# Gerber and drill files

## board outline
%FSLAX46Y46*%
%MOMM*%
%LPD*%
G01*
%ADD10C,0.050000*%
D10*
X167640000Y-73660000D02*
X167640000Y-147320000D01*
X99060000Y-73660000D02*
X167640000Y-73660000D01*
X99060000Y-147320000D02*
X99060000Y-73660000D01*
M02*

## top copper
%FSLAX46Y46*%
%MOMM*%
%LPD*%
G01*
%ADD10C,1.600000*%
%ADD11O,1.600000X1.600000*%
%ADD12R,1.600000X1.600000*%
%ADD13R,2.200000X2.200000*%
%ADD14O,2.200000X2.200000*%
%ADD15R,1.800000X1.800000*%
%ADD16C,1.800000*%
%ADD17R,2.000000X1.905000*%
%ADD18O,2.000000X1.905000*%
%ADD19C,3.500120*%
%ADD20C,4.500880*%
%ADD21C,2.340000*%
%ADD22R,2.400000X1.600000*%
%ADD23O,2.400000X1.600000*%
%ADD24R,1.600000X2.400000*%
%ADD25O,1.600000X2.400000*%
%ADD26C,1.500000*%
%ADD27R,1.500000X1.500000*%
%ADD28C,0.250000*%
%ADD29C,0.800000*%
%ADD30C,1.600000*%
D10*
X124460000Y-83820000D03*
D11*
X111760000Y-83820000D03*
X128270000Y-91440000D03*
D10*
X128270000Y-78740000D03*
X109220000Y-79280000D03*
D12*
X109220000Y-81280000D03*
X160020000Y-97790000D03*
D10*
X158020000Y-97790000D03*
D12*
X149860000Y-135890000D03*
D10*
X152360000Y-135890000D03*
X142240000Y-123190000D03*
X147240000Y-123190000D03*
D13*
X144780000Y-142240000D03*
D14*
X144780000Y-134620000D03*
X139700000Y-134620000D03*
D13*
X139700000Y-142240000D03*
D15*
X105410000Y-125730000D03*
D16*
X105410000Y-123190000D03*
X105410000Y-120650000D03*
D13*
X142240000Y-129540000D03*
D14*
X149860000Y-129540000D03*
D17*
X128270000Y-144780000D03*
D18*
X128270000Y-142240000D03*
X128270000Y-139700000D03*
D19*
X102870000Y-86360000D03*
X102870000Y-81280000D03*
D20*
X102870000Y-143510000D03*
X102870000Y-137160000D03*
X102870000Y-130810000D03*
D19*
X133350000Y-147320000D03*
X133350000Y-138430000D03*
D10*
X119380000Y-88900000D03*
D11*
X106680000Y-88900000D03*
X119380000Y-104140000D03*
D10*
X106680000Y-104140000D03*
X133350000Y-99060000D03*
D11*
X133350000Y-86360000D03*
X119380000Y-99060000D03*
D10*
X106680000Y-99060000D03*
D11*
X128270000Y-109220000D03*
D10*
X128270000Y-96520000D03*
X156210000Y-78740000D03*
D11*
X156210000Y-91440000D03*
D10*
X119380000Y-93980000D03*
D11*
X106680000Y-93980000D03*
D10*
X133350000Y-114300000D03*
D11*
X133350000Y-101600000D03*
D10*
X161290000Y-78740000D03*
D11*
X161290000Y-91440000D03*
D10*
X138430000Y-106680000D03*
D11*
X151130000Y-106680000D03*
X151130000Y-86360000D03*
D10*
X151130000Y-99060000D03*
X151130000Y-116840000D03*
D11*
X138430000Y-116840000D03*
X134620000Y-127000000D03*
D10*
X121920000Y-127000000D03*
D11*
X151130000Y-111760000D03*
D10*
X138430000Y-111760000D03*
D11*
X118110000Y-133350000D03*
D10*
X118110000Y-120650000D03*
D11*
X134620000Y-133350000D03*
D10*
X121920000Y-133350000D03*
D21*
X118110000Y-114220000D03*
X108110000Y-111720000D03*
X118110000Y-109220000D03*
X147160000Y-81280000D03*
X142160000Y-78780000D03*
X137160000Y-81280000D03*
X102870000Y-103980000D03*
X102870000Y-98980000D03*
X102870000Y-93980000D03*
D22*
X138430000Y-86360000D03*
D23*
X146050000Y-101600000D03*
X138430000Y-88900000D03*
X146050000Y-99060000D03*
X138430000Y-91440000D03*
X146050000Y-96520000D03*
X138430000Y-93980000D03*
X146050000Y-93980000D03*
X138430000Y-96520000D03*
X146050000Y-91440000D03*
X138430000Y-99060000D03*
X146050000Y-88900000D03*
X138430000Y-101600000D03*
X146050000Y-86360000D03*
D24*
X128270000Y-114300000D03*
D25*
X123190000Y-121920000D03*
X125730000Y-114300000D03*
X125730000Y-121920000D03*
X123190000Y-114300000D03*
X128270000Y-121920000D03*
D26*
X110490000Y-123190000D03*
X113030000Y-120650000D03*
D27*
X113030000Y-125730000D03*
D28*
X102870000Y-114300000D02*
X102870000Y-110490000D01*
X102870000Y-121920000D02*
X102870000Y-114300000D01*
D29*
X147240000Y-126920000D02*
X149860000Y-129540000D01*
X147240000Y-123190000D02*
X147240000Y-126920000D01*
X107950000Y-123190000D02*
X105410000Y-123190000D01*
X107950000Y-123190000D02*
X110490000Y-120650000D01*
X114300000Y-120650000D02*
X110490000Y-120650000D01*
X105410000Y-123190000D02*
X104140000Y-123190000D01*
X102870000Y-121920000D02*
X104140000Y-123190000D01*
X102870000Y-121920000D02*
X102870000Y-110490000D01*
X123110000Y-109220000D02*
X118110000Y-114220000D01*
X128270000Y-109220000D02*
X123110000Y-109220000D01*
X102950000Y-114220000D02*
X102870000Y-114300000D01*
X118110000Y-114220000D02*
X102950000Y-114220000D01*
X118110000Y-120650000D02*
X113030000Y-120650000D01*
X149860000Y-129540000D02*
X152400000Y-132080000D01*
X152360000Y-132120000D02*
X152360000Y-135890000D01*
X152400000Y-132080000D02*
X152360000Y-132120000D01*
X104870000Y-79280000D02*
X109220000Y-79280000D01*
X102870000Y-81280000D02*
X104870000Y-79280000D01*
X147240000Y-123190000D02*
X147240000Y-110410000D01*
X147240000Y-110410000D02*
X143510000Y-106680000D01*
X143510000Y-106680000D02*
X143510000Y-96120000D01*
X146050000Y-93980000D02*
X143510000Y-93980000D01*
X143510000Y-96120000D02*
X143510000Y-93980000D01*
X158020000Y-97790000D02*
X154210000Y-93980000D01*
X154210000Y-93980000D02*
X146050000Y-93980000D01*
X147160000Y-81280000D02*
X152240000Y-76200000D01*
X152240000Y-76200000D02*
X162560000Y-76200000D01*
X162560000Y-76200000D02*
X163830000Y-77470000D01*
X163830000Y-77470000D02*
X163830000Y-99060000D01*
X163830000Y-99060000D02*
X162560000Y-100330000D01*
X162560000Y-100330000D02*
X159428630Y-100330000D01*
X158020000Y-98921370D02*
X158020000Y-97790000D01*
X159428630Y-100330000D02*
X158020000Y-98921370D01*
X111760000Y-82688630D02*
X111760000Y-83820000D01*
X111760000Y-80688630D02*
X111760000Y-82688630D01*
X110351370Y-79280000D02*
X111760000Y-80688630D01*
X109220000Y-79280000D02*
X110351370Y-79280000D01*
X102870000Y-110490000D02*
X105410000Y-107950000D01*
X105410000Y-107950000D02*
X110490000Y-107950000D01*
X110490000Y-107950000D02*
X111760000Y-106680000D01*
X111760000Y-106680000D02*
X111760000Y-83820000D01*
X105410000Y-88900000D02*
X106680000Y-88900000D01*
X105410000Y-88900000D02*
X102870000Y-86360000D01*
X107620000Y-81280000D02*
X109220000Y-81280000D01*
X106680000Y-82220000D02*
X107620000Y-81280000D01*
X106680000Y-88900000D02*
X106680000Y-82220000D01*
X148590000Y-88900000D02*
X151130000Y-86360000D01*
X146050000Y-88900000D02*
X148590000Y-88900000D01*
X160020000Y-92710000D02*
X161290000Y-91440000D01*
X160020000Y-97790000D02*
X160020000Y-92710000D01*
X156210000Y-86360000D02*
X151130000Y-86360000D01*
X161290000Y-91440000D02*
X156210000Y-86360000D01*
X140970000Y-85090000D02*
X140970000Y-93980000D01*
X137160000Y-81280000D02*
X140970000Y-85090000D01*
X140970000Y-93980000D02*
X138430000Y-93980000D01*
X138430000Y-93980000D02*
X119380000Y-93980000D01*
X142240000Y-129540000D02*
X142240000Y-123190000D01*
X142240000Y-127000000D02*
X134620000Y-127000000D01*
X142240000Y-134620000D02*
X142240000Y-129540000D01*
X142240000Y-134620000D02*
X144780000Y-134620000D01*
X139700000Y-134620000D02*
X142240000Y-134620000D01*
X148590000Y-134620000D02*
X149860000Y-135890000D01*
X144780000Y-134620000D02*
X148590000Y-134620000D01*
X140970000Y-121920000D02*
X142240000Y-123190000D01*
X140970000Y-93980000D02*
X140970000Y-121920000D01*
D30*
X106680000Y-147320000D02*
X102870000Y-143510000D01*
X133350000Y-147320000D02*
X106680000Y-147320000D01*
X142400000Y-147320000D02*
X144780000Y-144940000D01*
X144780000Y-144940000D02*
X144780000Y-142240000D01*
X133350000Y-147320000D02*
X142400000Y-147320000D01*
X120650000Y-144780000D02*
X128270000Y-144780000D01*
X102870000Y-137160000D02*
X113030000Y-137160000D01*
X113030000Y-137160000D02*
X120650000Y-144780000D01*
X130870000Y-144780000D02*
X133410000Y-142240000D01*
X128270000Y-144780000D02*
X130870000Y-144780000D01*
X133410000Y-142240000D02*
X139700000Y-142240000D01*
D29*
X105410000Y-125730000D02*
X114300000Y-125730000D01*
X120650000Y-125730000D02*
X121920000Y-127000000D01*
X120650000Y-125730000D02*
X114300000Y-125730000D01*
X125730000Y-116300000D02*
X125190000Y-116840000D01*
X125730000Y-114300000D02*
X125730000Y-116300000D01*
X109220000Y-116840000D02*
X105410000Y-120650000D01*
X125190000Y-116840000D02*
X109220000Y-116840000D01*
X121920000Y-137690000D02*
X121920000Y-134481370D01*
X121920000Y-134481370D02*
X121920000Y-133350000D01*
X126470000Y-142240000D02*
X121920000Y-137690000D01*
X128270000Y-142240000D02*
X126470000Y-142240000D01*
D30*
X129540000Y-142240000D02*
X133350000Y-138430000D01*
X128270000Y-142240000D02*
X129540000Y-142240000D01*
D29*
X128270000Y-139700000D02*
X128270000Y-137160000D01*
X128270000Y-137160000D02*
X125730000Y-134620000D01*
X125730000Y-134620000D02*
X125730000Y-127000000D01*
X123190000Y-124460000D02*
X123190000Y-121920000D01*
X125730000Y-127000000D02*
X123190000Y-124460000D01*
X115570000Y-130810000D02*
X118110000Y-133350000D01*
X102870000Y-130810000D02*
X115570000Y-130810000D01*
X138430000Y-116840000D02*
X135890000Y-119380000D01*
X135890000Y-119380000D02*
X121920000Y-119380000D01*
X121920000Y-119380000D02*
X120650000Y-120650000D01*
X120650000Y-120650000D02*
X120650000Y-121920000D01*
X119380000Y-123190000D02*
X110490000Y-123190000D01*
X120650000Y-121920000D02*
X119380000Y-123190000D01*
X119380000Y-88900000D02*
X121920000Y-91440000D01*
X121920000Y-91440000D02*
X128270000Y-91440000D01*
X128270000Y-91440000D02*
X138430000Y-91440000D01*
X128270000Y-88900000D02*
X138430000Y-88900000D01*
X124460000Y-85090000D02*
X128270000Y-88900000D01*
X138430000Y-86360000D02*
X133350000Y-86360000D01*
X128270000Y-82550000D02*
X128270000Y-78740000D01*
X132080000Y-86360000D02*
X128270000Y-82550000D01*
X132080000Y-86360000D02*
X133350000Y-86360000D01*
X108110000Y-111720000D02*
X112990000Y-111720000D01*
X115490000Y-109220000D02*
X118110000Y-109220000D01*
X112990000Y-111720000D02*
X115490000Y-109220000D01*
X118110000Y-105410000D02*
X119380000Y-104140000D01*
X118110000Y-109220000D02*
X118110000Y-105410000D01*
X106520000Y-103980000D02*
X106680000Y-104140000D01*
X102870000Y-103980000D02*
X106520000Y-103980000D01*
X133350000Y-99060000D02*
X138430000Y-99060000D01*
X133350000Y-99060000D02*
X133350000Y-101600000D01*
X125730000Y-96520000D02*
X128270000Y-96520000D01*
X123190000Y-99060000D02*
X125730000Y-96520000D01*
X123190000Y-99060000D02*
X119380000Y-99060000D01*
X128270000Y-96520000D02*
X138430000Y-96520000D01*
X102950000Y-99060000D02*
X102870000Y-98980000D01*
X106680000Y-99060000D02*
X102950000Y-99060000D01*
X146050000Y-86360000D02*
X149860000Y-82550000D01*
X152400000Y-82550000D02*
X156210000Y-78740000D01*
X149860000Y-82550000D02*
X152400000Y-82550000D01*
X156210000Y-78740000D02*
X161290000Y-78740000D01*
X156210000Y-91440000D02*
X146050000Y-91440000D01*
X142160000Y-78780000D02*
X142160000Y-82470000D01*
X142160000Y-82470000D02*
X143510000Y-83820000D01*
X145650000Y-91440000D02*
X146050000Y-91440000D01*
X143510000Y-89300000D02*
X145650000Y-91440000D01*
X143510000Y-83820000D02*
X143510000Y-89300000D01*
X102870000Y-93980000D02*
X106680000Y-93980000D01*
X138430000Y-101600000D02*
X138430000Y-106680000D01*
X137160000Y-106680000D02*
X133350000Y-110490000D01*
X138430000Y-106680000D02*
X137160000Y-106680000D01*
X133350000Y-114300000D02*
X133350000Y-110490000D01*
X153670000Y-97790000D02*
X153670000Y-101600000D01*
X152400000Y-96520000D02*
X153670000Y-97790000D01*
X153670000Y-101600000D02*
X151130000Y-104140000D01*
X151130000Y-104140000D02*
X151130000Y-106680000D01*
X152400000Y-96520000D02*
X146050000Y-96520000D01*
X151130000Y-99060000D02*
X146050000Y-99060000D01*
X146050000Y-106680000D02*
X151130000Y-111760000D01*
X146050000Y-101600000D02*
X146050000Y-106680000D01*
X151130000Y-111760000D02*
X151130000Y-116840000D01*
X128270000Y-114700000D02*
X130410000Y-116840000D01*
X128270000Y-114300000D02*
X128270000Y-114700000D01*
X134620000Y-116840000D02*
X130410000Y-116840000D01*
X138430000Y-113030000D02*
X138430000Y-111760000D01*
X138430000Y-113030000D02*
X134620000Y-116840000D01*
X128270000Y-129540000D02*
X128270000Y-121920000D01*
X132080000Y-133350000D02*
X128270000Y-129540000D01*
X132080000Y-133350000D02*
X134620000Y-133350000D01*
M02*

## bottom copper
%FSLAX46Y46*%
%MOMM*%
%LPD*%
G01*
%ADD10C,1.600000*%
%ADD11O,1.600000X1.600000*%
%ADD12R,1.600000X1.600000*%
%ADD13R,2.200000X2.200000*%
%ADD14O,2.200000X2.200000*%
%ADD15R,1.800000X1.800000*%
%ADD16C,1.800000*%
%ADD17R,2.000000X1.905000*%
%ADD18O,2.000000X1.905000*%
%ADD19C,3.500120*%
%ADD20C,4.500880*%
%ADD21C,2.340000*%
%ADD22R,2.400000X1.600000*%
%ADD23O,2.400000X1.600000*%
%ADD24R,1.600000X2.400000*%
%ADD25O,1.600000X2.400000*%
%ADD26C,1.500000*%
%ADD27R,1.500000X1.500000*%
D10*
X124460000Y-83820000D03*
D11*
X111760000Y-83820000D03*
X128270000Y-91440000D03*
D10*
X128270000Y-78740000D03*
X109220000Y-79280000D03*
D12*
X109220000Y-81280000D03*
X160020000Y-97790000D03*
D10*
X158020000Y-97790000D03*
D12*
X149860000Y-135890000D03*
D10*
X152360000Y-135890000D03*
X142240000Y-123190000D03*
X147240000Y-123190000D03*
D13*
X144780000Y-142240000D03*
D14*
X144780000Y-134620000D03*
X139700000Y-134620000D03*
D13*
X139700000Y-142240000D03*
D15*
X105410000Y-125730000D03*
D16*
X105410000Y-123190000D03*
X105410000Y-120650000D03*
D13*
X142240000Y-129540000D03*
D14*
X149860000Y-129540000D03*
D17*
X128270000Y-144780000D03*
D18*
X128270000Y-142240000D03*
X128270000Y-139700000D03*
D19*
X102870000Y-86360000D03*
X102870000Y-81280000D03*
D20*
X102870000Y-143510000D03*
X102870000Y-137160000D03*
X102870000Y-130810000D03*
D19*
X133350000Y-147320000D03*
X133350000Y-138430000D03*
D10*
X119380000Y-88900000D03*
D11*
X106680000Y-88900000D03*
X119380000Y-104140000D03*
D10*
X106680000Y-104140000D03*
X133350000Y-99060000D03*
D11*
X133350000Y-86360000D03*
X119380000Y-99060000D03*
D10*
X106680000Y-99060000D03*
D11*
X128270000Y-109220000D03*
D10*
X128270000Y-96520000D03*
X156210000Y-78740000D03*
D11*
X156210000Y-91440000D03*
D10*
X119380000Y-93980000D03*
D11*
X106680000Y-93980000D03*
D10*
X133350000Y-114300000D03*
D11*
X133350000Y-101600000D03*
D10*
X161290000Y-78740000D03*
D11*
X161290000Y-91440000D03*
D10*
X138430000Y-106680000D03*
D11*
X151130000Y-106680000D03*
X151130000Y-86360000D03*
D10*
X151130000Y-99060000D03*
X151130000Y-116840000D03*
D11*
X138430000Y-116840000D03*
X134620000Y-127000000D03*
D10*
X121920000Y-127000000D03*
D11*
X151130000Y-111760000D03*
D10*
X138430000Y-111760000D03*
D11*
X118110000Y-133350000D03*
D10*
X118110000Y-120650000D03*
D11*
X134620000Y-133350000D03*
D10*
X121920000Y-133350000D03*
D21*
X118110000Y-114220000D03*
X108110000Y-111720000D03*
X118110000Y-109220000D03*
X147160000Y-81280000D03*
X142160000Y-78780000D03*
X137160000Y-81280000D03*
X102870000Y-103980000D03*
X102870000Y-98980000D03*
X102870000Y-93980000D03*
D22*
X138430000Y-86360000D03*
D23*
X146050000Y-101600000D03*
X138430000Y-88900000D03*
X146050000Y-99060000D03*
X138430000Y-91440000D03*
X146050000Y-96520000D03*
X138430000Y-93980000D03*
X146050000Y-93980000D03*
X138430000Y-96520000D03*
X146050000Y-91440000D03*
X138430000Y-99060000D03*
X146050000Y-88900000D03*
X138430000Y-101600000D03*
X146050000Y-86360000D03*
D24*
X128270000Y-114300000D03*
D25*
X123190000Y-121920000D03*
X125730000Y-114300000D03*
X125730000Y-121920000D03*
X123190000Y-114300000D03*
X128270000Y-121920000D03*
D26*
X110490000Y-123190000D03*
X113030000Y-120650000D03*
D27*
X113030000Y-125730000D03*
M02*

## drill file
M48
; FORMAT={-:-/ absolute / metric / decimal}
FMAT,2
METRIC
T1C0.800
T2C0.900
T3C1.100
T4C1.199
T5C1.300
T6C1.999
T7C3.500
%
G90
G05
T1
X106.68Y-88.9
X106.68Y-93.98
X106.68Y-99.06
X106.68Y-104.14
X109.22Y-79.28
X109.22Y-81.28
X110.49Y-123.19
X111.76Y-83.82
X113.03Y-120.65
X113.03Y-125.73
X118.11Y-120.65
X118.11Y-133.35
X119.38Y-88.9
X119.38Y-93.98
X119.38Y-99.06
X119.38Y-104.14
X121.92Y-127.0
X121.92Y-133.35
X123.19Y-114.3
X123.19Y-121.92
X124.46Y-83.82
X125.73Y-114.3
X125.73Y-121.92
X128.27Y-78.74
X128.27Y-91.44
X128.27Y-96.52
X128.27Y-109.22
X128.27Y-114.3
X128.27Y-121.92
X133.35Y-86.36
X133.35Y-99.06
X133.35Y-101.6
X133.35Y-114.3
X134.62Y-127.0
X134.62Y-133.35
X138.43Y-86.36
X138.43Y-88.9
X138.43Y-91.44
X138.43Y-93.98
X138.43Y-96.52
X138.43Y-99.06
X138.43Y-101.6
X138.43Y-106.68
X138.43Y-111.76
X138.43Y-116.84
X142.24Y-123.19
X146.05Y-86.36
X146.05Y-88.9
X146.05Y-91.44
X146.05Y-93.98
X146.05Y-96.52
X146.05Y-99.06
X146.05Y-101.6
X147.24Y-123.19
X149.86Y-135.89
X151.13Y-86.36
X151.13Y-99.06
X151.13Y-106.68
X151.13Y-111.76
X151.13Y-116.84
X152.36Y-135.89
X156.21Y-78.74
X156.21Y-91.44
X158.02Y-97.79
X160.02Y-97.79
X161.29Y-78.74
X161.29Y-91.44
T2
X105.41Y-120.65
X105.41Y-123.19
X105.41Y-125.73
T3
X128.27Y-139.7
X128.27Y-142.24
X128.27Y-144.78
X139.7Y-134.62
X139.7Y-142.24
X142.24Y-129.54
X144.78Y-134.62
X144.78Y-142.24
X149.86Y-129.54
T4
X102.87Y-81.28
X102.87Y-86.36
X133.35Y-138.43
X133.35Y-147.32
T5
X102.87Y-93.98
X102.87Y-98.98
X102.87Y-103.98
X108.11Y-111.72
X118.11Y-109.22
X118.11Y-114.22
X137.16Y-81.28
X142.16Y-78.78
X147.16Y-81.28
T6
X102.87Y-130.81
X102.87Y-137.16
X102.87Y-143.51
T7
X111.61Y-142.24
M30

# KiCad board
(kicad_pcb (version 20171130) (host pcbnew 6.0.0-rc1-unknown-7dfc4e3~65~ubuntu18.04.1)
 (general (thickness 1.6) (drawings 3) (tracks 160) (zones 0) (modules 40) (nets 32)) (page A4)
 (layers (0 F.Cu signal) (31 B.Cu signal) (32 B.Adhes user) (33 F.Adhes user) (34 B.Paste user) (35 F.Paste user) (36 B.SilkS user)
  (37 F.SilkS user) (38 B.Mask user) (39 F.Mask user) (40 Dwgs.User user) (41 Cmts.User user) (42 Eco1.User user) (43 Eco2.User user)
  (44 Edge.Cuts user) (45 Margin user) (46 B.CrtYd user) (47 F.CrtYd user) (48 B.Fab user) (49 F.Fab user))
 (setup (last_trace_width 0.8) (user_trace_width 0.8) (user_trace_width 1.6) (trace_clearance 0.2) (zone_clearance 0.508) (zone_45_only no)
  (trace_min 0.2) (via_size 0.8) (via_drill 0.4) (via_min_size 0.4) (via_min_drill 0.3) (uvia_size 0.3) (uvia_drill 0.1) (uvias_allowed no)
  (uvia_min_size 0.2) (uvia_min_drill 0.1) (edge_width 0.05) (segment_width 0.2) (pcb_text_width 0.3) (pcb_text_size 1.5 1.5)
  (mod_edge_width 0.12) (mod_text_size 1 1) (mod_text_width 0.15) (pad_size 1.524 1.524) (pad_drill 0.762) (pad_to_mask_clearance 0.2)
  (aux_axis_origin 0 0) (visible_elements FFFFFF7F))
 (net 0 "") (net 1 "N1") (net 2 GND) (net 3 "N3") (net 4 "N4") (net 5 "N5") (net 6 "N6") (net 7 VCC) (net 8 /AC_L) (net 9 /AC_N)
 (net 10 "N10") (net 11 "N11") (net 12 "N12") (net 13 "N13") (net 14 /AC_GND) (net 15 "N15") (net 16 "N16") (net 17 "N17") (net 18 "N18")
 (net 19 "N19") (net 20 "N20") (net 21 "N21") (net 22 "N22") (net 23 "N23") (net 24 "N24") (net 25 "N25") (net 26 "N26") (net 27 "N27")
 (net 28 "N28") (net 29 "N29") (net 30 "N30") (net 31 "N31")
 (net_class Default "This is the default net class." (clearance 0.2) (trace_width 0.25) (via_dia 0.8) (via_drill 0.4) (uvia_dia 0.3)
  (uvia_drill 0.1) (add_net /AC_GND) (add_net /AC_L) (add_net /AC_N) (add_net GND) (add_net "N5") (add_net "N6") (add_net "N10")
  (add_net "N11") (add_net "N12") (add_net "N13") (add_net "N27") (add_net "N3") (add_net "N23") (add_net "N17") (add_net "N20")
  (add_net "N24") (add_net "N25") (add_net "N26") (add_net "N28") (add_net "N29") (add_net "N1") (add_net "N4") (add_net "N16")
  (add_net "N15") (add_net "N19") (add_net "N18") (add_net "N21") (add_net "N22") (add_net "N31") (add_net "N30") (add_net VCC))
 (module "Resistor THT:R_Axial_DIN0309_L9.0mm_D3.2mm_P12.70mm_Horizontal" (layer F.Cu) (at 124.46 83.82 180)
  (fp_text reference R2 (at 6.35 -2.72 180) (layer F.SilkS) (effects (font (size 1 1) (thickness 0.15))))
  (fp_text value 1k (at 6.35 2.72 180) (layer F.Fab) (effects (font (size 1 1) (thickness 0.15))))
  (pad 1 thru_hole circle (at 0 0 180) (size 1.6 1.6) (drill 0.8) (layers *.Cu *.Mask) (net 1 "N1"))
  (pad 2 thru_hole oval (at 12.7 0 180) (size 1.6 1.6) (drill 0.8) (layers *.Cu *.Mask) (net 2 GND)))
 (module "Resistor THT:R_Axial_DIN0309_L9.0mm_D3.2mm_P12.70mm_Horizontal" (layer F.Cu) (at 128.27 78.74 270)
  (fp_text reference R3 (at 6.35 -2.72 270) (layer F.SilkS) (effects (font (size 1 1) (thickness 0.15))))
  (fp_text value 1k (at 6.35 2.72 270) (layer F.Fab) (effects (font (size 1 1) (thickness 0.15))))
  (pad 2 thru_hole oval (at 12.7 0 270) (size 1.6 1.6) (drill 0.8) (layers *.Cu *.Mask) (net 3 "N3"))
  (pad 1 thru_hole circle (at 0 0 270) (size 1.6 1.6) (drill 0.8) (layers *.Cu *.Mask) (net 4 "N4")))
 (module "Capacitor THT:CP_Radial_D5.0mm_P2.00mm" (layer F.Cu) (at 109.22 81.28 90)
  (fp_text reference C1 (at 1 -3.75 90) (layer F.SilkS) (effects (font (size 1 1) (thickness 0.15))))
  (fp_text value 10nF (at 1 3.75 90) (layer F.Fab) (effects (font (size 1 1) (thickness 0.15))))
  (pad 2 thru_hole circle (at 2 0 90) (size 1.6 1.6) (drill 0.8) (layers *.Cu *.Mask) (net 2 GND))
  (pad 1 thru_hole rect (at 0 0 90) (size 1.6 1.6) (drill 0.8) (layers *.Cu *.Mask) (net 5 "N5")))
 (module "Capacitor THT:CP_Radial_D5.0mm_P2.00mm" (layer F.Cu) (at 160.02 97.79 180)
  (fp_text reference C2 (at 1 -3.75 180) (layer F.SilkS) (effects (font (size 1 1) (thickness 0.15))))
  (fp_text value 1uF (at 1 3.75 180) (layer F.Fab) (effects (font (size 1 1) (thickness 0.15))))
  (pad 1 thru_hole rect (at 0 0 180) (size 1.6 1.6) (drill 0.8) (layers *.Cu *.Mask) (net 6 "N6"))
  (pad 2 thru_hole circle (at 2 0 180) (size 1.6 1.6) (drill 0.8) (layers *.Cu *.Mask) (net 2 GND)))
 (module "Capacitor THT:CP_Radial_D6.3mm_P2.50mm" (layer F.Cu) (at 149.86 135.89)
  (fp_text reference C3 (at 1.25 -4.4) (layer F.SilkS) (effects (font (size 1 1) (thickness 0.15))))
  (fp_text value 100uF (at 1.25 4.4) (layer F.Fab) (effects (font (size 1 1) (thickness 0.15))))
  (pad 1 thru_hole rect (at 0 0) (size 1.6 1.6) (drill 0.8) (layers *.Cu *.Mask) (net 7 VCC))
  (pad 2 thru_hole circle (at 2.5 0) (size 1.6 1.6) (drill 0.8) (layers *.Cu *.Mask) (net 2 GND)))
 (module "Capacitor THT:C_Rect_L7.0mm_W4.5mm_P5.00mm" (layer F.Cu) (at 142.24 123.19)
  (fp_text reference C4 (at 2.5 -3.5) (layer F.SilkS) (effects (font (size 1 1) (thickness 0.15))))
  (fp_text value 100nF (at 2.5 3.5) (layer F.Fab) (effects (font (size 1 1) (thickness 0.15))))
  (pad 1 thru_hole circle (at 0 0) (size 1.6 1.6) (drill 0.8) (layers *.Cu *.Mask) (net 7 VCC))
  (pad 2 thru_hole circle (at 5 0) (size 1.6 1.6) (drill 0.8) (layers *.Cu *.Mask) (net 2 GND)))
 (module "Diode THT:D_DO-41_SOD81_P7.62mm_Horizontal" (layer F.Cu) (at 144.78 142.24 90)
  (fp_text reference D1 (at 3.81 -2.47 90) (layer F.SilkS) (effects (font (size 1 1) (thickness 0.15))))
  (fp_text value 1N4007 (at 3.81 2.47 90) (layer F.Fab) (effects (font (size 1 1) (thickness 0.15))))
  (pad 1 thru_hole rect (at 0 0 90) (size 2.2 2.2) (drill 1.1) (layers *.Cu *.Mask) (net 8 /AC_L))
  (pad 2 thru_hole oval (at 7.62 0 90) (size 2.2 2.2) (drill 1.1) (layers *.Cu *.Mask) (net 7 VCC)))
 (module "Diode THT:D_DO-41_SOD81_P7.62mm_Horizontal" (layer F.Cu) (at 139.7 142.24 90)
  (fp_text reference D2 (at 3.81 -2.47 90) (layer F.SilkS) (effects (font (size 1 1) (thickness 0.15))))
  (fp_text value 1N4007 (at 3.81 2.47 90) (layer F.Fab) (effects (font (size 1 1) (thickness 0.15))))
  (pad 2 thru_hole oval (at 7.62 0 90) (size 2.2 2.2) (drill 1.1) (layers *.Cu *.Mask) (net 7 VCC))
  (pad 1 thru_hole rect (at 0 0 90) (size 2.2 2.2) (drill 1.1) (layers *.Cu *.Mask) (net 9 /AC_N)))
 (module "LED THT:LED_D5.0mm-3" (layer F.Cu) (at 105.41 125.73 90)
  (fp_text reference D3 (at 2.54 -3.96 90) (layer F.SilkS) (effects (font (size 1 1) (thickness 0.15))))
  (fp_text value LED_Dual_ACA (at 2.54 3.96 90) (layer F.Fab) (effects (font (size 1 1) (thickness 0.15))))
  (pad 1 thru_hole rect (at 0 0 90) (size 1.8 1.8) (drill 0.9) (layers *.Cu *.Mask) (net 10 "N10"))
  (pad 2 thru_hole circle (at 2.54 0 90) (size 1.8 1.8) (drill 0.9) (layers *.Cu *.Mask) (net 2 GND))
  (pad 3 thru_hole circle (at 5.08 0 90) (size 1.8 1.8) (drill 0.9) (layers *.Cu *.Mask) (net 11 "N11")))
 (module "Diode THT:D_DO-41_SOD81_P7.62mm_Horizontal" (layer F.Cu) (at 142.24 129.54)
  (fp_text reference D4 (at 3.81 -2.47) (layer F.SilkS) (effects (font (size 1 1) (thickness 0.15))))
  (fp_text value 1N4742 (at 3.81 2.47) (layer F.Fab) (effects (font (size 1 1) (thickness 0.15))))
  (pad 1 thru_hole rect (at 0 0) (size 2.2 2.2) (drill 1.1) (layers *.Cu *.Mask) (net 7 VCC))
  (pad 2 thru_hole oval (at 7.62 0) (size 2.2 2.2) (drill 1.1) (layers *.Cu *.Mask) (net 2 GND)))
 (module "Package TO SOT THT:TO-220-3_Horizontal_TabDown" (layer F.Cu) (at 128.27 144.78 90)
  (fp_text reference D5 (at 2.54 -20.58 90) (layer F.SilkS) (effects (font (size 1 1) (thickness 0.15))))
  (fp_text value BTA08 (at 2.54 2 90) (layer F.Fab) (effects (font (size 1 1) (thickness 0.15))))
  (pad "" np_thru_hole oval (at 2.54 -16.66 90) (size 3.5 3.5) (drill 3.5) (layers *.Cu *.Mask))
  (pad 1 thru_hole rect (at 0 0 90) (size 1.905 2) (drill 1.1) (layers *.Cu *.Mask) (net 9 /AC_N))
  (pad 2 thru_hole oval (at 2.54 0 90) (size 1.905 2) (drill 1.1) (layers *.Cu *.Mask) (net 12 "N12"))
  (pad 3 thru_hole oval (at 5.08 0 90) (size 1.905 2) (drill 1.1) (layers *.Cu *.Mask) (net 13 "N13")))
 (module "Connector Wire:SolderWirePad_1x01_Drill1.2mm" (layer F.Cu) (at 102.87 86.36)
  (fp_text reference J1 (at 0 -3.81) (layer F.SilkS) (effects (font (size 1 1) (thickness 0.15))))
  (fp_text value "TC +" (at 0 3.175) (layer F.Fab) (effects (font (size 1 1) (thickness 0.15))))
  (pad 1 thru_hole circle (at 0 0) (size 3.50012 3.50012) (drill 1.19888) (layers *.Cu *.Mask) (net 5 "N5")))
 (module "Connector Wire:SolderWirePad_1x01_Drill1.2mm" (layer F.Cu) (at 102.87 81.28)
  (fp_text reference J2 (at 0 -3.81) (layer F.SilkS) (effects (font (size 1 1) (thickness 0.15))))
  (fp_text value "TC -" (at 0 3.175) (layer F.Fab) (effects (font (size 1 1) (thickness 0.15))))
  (pad 1 thru_hole circle (at 0 0) (size 3.50012 3.50012) (drill 1.19888) (layers *.Cu *.Mask) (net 2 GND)))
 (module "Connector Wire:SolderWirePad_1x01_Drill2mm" (layer F.Cu) (at 102.87 143.51 180)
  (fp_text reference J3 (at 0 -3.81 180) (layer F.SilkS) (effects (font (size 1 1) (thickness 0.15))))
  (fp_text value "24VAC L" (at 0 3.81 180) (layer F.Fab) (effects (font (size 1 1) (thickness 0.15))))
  (pad 1 thru_hole circle (at 0 0 180) (size 4.50088 4.50088) (drill 1.99898) (layers *.Cu *.Mask) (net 8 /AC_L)))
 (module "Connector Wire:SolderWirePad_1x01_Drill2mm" (layer F.Cu) (at 102.87 137.16 180)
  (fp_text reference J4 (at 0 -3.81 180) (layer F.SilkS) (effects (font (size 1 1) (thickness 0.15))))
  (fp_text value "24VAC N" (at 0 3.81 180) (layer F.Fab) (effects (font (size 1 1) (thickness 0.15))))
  (pad 1 thru_hole circle (at 0 0 180) (size 4.50088 4.50088) (drill 1.99898) (layers *.Cu *.Mask) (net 9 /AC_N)))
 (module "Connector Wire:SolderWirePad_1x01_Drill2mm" (layer F.Cu) (at 102.87 130.81 180)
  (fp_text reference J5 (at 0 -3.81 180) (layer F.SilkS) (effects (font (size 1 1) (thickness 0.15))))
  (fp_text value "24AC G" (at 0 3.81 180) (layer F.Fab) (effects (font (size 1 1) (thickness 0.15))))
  (pad 1 thru_hole circle (at 0 0 180) (size 4.50088 4.50088) (drill 1.99898) (layers *.Cu *.Mask) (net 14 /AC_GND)))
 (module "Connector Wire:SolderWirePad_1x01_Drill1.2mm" (layer F.Cu) (at 133.35 147.32)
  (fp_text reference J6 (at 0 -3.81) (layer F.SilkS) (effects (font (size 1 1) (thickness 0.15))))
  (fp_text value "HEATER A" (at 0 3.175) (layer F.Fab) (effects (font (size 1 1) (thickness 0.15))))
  (pad 1 thru_hole circle (at 0 0) (size 3.50012 3.50012) (drill 1.19888) (layers *.Cu *.Mask) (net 8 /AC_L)))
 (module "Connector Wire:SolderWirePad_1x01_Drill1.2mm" (layer F.Cu) (at 133.35 138.43)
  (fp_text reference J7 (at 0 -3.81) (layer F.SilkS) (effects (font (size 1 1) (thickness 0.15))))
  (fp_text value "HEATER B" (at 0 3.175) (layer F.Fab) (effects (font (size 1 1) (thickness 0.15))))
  (pad 1 thru_hole circle (at 0 0) (size 3.50012 3.50012) (drill 1.19888) (layers *.Cu *.Mask) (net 12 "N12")))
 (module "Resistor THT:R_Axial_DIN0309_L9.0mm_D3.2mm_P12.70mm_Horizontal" (layer F.Cu) (at 119.38 88.9 180)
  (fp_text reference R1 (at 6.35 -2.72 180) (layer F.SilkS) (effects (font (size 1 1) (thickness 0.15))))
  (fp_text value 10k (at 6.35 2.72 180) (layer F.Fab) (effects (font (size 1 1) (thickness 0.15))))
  (pad 1 thru_hole circle (at 0 0 180) (size 1.6 1.6) (drill 0.8) (layers *.Cu *.Mask) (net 3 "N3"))
  (pad 2 thru_hole oval (at 12.7 0 180) (size 1.6 1.6) (drill 0.8) (layers *.Cu *.Mask) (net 5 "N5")))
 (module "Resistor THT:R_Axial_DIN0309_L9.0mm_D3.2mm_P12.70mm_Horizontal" (layer F.Cu) (at 106.68 104.14)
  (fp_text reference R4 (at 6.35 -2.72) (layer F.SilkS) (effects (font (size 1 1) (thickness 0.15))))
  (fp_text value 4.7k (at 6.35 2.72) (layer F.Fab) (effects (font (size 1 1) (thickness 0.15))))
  (pad 2 thru_hole oval (at 12.7 0) (size 1.6 1.6) (drill 0.8) (layers *.Cu *.Mask) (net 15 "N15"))
  (pad 1 thru_hole circle (at 0 0) (size 1.6 1.6) (drill 0.8) (layers *.Cu *.Mask) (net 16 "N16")))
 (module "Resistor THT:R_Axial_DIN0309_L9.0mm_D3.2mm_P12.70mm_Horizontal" (layer F.Cu) (at 133.35 99.06 90)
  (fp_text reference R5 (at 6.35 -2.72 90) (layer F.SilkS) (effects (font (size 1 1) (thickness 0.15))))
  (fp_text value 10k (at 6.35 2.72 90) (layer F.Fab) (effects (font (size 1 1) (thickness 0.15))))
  (pad 1 thru_hole circle (at 0 0 90) (size 1.6 1.6) (drill 0.8) (layers *.Cu *.Mask) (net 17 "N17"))
  (pad 2 thru_hole oval (at 12.7 0 90) (size 1.6 1.6) (drill 0.8) (layers *.Cu *.Mask) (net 4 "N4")))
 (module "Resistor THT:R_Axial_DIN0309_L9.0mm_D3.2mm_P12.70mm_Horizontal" (layer F.Cu) (at 106.68 99.06)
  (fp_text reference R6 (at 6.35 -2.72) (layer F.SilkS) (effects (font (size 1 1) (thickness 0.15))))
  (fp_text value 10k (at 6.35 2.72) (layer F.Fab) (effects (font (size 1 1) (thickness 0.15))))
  (pad 2 thru_hole oval (at 12.7 0) (size 1.6 1.6) (drill 0.8) (layers *.Cu *.Mask) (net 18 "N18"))
  (pad 1 thru_hole circle (at 0 0) (size 1.6 1.6) (drill 0.8) (layers *.Cu *.Mask) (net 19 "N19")))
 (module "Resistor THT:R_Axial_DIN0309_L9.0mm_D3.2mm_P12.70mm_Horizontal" (layer F.Cu) (at 128.27 96.52 270)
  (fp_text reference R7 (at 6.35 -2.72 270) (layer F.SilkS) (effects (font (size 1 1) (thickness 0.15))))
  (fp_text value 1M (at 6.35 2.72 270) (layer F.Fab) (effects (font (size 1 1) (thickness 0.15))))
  (pad 2 thru_hole oval (at 12.7 0 270) (size 1.6 1.6) (drill 0.8) (layers *.Cu *.Mask) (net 2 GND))
  (pad 1 thru_hole circle (at 0 0 270) (size 1.6 1.6) (drill 0.8) (layers *.Cu *.Mask) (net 18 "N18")))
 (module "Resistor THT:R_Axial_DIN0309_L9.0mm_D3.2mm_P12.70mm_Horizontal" (layer F.Cu) (at 156.21 78.74 270)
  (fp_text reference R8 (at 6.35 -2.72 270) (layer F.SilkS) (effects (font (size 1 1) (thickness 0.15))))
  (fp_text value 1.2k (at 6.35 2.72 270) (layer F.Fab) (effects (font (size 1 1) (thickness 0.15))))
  (pad 1 thru_hole circle (at 0 0 270) (size 1.6 1.6) (drill 0.8) (layers *.Cu *.Mask) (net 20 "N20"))
  (pad 2 thru_hole oval (at 12.7 0 270) (size 1.6 1.6) (drill 0.8) (layers *.Cu *.Mask) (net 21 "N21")))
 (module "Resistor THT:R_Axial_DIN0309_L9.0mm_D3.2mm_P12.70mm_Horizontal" (layer F.Cu) (at 119.38 93.98 180)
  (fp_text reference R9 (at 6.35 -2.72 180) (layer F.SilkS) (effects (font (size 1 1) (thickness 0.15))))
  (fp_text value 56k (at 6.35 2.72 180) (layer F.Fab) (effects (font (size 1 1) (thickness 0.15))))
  (pad 1 thru_hole circle (at 0 0 180) (size 1.6 1.6) (drill 0.8) (layers *.Cu *.Mask) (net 7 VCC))
  (pad 2 thru_hole oval (at 12.7 0 180) (size 1.6 1.6) (drill 0.8) (layers *.Cu *.Mask) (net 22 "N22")))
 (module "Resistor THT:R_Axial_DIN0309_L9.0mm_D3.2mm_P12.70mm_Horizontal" (layer F.Cu) (at 133.35 114.3 90)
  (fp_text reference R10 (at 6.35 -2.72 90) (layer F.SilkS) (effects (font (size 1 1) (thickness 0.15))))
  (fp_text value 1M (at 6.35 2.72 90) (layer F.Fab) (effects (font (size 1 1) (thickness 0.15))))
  (pad 1 thru_hole circle (at 0 0 90) (size 1.6 1.6) (drill 0.8) (layers *.Cu *.Mask) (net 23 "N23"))
  (pad 2 thru_hole oval (at 12.7 0 90) (size 1.6 1.6) (drill 0.8) (layers *.Cu *.Mask) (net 17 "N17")))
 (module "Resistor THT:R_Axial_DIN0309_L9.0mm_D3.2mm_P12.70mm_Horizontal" (layer F.Cu) (at 161.29 78.74 270)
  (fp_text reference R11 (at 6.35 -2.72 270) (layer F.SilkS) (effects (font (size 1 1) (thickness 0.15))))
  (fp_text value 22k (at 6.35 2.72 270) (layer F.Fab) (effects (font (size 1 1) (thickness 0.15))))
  (pad 1 thru_hole circle (at 0 0 270) (size 1.6 1.6) (drill 0.8) (layers *.Cu *.Mask) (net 20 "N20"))
  (pad 2 thru_hole oval (at 12.7 0 270) (size 1.6 1.6) (drill 0.8) (layers *.Cu *.Mask) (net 6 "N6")))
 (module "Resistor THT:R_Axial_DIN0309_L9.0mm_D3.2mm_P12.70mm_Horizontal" (layer F.Cu) (at 138.43 106.68)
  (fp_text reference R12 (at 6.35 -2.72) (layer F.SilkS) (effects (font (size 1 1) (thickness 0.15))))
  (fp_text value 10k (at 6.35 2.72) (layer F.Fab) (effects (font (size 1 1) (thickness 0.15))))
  (pad 1 thru_hole circle (at 0 0) (size 1.6 1.6) (drill 0.8) (layers *.Cu *.Mask) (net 23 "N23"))
  (pad 2 thru_hole oval (at 12.7 0) (size 1.6 1.6) (drill 0.8) (layers *.Cu *.Mask) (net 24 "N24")))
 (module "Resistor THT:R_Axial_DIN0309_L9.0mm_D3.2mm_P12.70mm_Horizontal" (layer F.Cu) (at 151.13 99.06 90)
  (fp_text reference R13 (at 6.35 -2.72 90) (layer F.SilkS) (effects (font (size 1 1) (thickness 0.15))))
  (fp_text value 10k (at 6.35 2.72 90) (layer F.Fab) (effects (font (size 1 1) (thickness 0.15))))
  (pad 2 thru_hole oval (at 12.7 0 90) (size 1.6 1.6) (drill 0.8) (layers *.Cu *.Mask) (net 6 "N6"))
  (pad 1 thru_hole circle (at 0 0 90) (size 1.6 1.6) (drill 0.8) (layers *.Cu *.Mask) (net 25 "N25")))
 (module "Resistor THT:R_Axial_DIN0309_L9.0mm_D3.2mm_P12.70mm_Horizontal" (layer F.Cu) (at 151.13 116.84 180)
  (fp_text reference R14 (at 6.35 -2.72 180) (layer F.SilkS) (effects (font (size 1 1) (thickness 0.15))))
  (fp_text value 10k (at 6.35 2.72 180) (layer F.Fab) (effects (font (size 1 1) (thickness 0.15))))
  (pad 1 thru_hole circle (at 0 0 180) (size 1.6 1.6) (drill 0.8) (layers *.Cu *.Mask) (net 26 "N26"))
  (pad 2 thru_hole oval (at 12.7 0 180) (size 1.6 1.6) (drill 0.8) (layers *.Cu *.Mask) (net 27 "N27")))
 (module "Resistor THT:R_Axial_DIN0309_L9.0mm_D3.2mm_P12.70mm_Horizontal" (layer F.Cu) (at 121.92 127)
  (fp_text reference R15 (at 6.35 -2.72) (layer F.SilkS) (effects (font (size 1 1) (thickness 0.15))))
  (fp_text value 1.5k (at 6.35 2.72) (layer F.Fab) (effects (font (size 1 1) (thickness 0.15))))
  (pad 2 thru_hole oval (at 12.7 0) (size 1.6 1.6) (drill 0.8) (layers *.Cu *.Mask) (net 7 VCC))
  (pad 1 thru_hole circle (at 0 0) (size 1.6 1.6) (drill 0.8) (layers *.Cu *.Mask) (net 10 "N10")))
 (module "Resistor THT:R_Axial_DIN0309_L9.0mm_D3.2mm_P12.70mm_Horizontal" (layer F.Cu) (at 138.43 111.76)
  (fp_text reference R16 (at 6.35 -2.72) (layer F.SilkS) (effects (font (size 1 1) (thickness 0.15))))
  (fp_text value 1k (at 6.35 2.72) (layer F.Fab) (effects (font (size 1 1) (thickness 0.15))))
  (pad 2 thru_hole oval (at 12.7 0) (size 1.6 1.6) (drill 0.8) (layers *.Cu *.Mask) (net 26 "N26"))
  (pad 1 thru_hole circle (at 0 0) (size 1.6 1.6) (drill 0.8) (layers *.Cu *.Mask) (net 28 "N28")))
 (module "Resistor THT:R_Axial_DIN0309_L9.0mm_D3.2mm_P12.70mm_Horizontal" (layer F.Cu) (at 118.11 120.65 270)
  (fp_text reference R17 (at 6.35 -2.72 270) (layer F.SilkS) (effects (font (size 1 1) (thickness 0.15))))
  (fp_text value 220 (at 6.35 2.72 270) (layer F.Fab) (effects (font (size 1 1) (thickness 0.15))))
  (pad 2 thru_hole oval (at 12.7 0 270) (size 1.6 1.6) (drill 0.8) (layers *.Cu *.Mask) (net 14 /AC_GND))
  (pad 1 thru_hole circle (at 0 0 270) (size 1.6 1.6) (drill 0.8) (layers *.Cu *.Mask) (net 2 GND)))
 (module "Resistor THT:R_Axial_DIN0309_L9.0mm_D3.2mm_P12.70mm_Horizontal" (layer F.Cu) (at 121.92 133.35)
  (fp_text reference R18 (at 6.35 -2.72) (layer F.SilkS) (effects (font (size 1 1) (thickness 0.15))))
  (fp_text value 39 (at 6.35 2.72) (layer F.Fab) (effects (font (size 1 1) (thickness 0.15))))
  (pad 2 thru_hole oval (at 12.7 0) (size 1.6 1.6) (drill 0.8) (layers *.Cu *.Mask) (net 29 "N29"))
  (pad 1 thru_hole circle (at 0 0) (size 1.6 1.6) (drill 0.8) (layers *.Cu *.Mask) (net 12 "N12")))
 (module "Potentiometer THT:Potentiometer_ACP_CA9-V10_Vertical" (layer F.Cu) (at 118.11 109.22 180)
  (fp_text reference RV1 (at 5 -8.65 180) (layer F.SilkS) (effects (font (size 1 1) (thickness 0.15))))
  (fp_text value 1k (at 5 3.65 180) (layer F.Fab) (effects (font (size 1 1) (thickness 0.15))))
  (pad 3 thru_hole circle (at 0 -5 180) (size 2.34 2.34) (drill 1.3) (layers *.Cu *.Mask) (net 2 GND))
  (pad 2 thru_hole circle (at 10 -2.5 180) (size 2.34 2.34) (drill 1.3) (layers *.Cu *.Mask) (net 15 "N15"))
  (pad 1 thru_hole circle (at 0 0 180) (size 2.34 2.34) (drill 1.3) (layers *.Cu *.Mask) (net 15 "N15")))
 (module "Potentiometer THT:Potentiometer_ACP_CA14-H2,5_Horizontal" (layer F.Cu) (at 137.16 81.28 90)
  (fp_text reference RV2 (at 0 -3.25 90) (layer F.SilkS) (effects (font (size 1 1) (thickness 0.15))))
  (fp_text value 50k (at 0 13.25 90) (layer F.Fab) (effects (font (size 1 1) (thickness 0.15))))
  (pad 3 thru_hole circle (at 0 10 90) (size 2.34 2.34) (drill 1.3) (layers *.Cu *.Mask) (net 2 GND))
  (pad 2 thru_hole circle (at 2.5 5 90) (size 2.34 2.34) (drill 1.3) (layers *.Cu *.Mask) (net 21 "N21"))
  (pad 1 thru_hole circle (at 0 0 90) (size 2.34 2.34) (drill 1.3) (layers *.Cu *.Mask) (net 7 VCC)))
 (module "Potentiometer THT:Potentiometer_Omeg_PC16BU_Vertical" (layer F.Cu) (at 102.87 93.98 180)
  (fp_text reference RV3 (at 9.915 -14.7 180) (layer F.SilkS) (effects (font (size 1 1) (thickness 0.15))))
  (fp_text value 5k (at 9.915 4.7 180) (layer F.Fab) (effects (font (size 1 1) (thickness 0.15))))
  (pad 3 thru_hole circle (at 0 -10 180) (size 2.34 2.34) (drill 1.3) (layers *.Cu *.Mask) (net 16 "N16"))
  (pad 2 thru_hole circle (at 0 -5 180) (size 2.34 2.34) (drill 1.3) (layers *.Cu *.Mask) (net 19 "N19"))
  (pad 1 thru_hole circle (at 0 0 180) (size 2.34 2.34) (drill 1.3) (layers *.Cu *.Mask) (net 22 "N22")))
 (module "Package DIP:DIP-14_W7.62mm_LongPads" (layer F.Cu) (at 138.43 86.36)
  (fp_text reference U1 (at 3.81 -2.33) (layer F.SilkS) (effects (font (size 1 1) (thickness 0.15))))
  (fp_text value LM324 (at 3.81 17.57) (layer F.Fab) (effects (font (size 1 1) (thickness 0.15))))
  (pad 1 thru_hole rect (at 0 0) (size 2.4 1.6) (drill 0.8) (layers *.Cu *.Mask) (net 4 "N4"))
  (pad 8 thru_hole oval (at 7.62 15.24) (size 2.4 1.6) (drill 0.8) (layers *.Cu *.Mask) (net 26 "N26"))
  (pad 2 thru_hole oval (at 0 2.54) (size 2.4 1.6) (drill 0.8) (layers *.Cu *.Mask) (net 1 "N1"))
  (pad 9 thru_hole oval (at 7.62 12.7) (size 2.4 1.6) (drill 0.8) (layers *.Cu *.Mask) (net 25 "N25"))
  (pad 3 thru_hole oval (at 0 5.08) (size 2.4 1.6) (drill 0.8) (layers *.Cu *.Mask) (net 3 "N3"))
  (pad 10 thru_hole oval (at 7.62 10.16) (size 2.4 1.6) (drill 0.8) (layers *.Cu *.Mask) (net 24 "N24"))
  (pad 4 thru_hole oval (at 0 7.62) (size 2.4 1.6) (drill 0.8) (layers *.Cu *.Mask) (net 7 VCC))
  (pad 11 thru_hole oval (at 7.62 7.62) (size 2.4 1.6) (drill 0.8) (layers *.Cu *.Mask) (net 2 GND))
  (pad 5 thru_hole oval (at 0 10.16) (size 2.4 1.6) (drill 0.8) (layers *.Cu *.Mask) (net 18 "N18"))
  (pad 12 thru_hole oval (at 7.62 5.08) (size 2.4 1.6) (drill 0.8) (layers *.Cu *.Mask) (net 21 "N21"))
  (pad 6 thru_hole oval (at 0 12.7) (size 2.4 1.6) (drill 0.8) (layers *.Cu *.Mask) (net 17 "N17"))
  (pad 13 thru_hole oval (at 7.62 2.54) (size 2.4 1.6) (drill 0.8) (layers *.Cu *.Mask) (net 6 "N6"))
  (pad 7 thru_hole oval (at 0 15.24) (size 2.4 1.6) (drill 0.8) (layers *.Cu *.Mask) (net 23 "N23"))
  (pad 14 thru_hole oval (at 7.62 0) (size 2.4 1.6) (drill 0.8) (layers *.Cu *.Mask) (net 20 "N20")))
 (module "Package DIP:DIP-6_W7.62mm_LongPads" (layer F.Cu) (at 128.27 114.3 270)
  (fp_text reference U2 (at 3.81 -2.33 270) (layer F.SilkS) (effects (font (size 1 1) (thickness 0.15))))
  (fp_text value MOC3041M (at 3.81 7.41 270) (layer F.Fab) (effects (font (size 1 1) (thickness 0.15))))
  (pad 1 thru_hole rect (at 0 0 270) (size 2.4 1.6) (drill 0.8) (layers *.Cu *.Mask) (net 28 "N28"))
  (pad 4 thru_hole oval (at 7.62 5.08 270) (size 2.4 1.6) (drill 0.8) (layers *.Cu *.Mask) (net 13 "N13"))
  (pad 2 thru_hole oval (at 0 2.54 270) (size 2.4 1.6) (drill 0.8) (layers *.Cu *.Mask) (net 11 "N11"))
  (pad 5 thru_hole oval (at 7.62 2.54 270) (size 2.4 1.6) (drill 0.8) (layers *.Cu *.Mask) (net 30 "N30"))
  (pad 3 thru_hole oval (at 0 5.08 270) (size 2.4 1.6) (drill 0.8) (layers *.Cu *.Mask) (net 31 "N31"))
  (pad 6 thru_hole oval (at 7.62 0 270) (size 2.4 1.6) (drill 0.8) (layers *.Cu *.Mask) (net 29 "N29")))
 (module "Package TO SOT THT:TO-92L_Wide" (layer F.Cu) (at 113.03 125.73 90)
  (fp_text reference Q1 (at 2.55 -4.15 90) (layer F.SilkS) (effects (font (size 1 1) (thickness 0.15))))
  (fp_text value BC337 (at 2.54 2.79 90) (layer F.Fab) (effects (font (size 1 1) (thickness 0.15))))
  (pad 2 thru_hole circle (at 2.54 -2.54 180) (size 1.5 1.5) (drill 0.8) (layers *.Cu *.Mask) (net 27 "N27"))
  (pad 3 thru_hole circle (at 5.08 0 180) (size 1.5 1.5) (drill 0.8) (layers *.Cu *.Mask) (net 2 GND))
  (pad 1 thru_hole rect (at 0 0 180) (size 1.5 1.5) (drill 0.8) (layers *.Cu *.Mask) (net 10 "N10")))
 (gr_line (start 167.64 73.66) (end 167.64 147.32) (layer Edge.Cuts) (width 0.05))
 (gr_line (start 99.06 73.66) (end 167.64 73.66) (layer Edge.Cuts) (width 0.05))
 (gr_line (start 99.06 147.32) (end 99.06 73.66) (layer Edge.Cuts) (width 0.05))
 (segment (start 102.87 114.3) (end 102.87 110.49) (width 0.25) (layer F.Cu) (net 2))
 (segment (start 102.87 121.92) (end 102.87 114.3) (width 0.25) (layer F.Cu) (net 2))
 (segment (start 147.24 126.92) (end 149.86 129.54) (width 0.8) (layer F.Cu) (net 2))
 (segment (start 147.24 123.19) (end 147.24 126.92) (width 0.8) (layer F.Cu) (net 2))
 (segment (start 107.95 123.19) (end 105.41 123.19) (width 0.8) (layer F.Cu) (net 2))
 (segment (start 107.95 123.19) (end 110.49 120.65) (width 0.8) (layer F.Cu) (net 2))
 (segment (start 114.3 120.65) (end 110.49 120.65) (width 0.8) (layer F.Cu) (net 2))
 (segment (start 105.41 123.19) (end 104.14 123.19) (width 0.8) (layer F.Cu) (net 2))
 (segment (start 102.87 121.92) (end 104.14 123.19) (width 0.8) (layer F.Cu) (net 2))
 (segment (start 102.87 121.92) (end 102.87 110.49) (width 0.8) (layer F.Cu) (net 2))
 (segment (start 123.11 109.22) (end 118.11 114.22) (width 0.8) (layer F.Cu) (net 2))
 (segment (start 128.27 109.22) (end 123.11 109.22) (width 0.8) (layer F.Cu) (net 2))
 (segment (start 102.95 114.22) (end 102.87 114.3) (width 0.8) (layer F.Cu) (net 2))
 (segment (start 118.11 114.22) (end 102.95 114.22) (width 0.8) (layer F.Cu) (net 2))
 (segment (start 118.11 120.65) (end 113.03 120.65) (width 0.8) (layer F.Cu) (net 2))
 (segment (start 149.86 129.54) (end 152.4 132.08) (width 0.8) (layer F.Cu) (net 2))
 (segment (start 152.36 132.12) (end 152.36 135.89) (width 0.8) (layer F.Cu) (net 2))
 (segment (start 152.4 132.08) (end 152.36 132.12) (width 0.8) (layer F.Cu) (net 2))
 (segment (start 104.87 79.28) (end 109.22 79.28) (width 0.8) (layer F.Cu) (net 2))
 (segment (start 102.87 81.28) (end 104.87 79.28) (width 0.8) (layer F.Cu) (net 2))
 (segment (start 147.24 123.19) (end 147.24 110.41) (width 0.8) (layer F.Cu) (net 2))
 (segment (start 147.24 110.41) (end 143.51 106.68) (width 0.8) (layer F.Cu) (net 2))
 (segment (start 143.51 106.68) (end 143.51 96.12) (width 0.8) (layer F.Cu) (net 2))
 (segment (start 146.05 93.98) (end 143.51 93.98) (width 0.8) (layer F.Cu) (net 2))
 (segment (start 143.51 96.12) (end 143.51 93.98) (width 0.8) (layer F.Cu) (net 2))
 (segment (start 158.02 97.79) (end 154.21 93.98) (width 0.8) (layer F.Cu) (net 2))
 (segment (start 154.21 93.98) (end 146.05 93.98) (width 0.8) (layer F.Cu) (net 2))
 (segment (start 147.16 81.28) (end 152.24 76.2) (width 0.8) (layer F.Cu) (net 2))
 (segment (start 152.24 76.2) (end 162.56 76.2) (width 0.8) (layer F.Cu) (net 2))
 (segment (start 162.56 76.2) (end 163.83 77.47) (width 0.8) (layer F.Cu) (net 2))
 (segment (start 163.83 77.47) (end 163.83 99.06) (width 0.8) (layer F.Cu) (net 2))
 (segment (start 163.83 99.06) (end 162.56 100.33) (width 0.8) (layer F.Cu) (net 2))
 (segment (start 162.56 100.33) (end 159.42863 100.33) (width 0.8) (layer F.Cu) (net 2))
 (segment (start 158.02 98.92137) (end 158.02 97.79) (width 0.8) (layer F.Cu) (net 2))
 (segment (start 159.42863 100.33) (end 158.02 98.92137) (width 0.8) (layer F.Cu) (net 2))
 (segment (start 111.76 82.68863) (end 111.76 83.82) (width 0.8) (layer F.Cu) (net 2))
 (segment (start 111.76 80.68863) (end 111.76 82.68863) (width 0.8) (layer F.Cu) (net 2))
 (segment (start 110.35137 79.28) (end 111.76 80.68863) (width 0.8) (layer F.Cu) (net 2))
 (segment (start 109.22 79.28) (end 110.35137 79.28) (width 0.8) (layer F.Cu) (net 2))
 (segment (start 102.87 110.49) (end 105.41 107.95) (width 0.8) (layer F.Cu) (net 2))
 (segment (start 105.41 107.95) (end 110.49 107.95) (width 0.8) (layer F.Cu) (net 2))
 (segment (start 110.49 107.95) (end 111.76 106.68) (width 0.8) (layer F.Cu) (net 2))
 (segment (start 111.76 106.68) (end 111.76 83.82) (width 0.8) (layer F.Cu) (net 2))
 (segment (start 105.41 88.9) (end 106.68 88.9) (width 0.8) (layer F.Cu) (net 5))
 (segment (start 105.41 88.9) (end 102.87 86.36) (width 0.8) (layer F.Cu) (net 5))
 (segment (start 107.62 81.28) (end 109.22 81.28) (width 0.8) (layer F.Cu) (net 5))
 (segment (start 106.68 82.22) (end 107.62 81.28) (width 0.8) (layer F.Cu) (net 5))
 (segment (start 106.68 88.9) (end 106.68 82.22) (width 0.8) (layer F.Cu) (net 5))
 (segment (start 148.59 88.9) (end 151.13 86.36) (width 0.8) (layer F.Cu) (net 6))
 (segment (start 146.05 88.9) (end 148.59 88.9) (width 0.8) (layer F.Cu) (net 6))
 (segment (start 160.02 92.71) (end 161.29 91.44) (width 0.8) (layer F.Cu) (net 6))
 (segment (start 160.02 97.79) (end 160.02 92.71) (width 0.8) (layer F.Cu) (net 6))
 (segment (start 156.21 86.36) (end 151.13 86.36) (width 0.8) (layer F.Cu) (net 6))
 (segment (start 161.29 91.44) (end 156.21 86.36) (width 0.8) (layer F.Cu) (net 6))
 (segment (start 140.97 85.09) (end 140.97 93.98) (width 0.8) (layer F.Cu) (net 7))
 (segment (start 137.16 81.28) (end 140.97 85.09) (width 0.8) (layer F.Cu) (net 7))
 (segment (start 140.97 93.98) (end 138.43 93.98) (width 0.8) (layer F.Cu) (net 7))
 (segment (start 138.43 93.98) (end 119.38 93.98) (width 0.8) (layer F.Cu) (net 7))
 (segment (start 142.24 129.54) (end 142.24 123.19) (width 0.8) (layer F.Cu) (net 7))
 (segment (start 142.24 127) (end 134.62 127) (width 0.8) (layer F.Cu) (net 7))
 (segment (start 142.24 134.62) (end 142.24 129.54) (width 0.8) (layer F.Cu) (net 7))
 (segment (start 142.24 134.62) (end 144.78 134.62) (width 0.8) (layer F.Cu) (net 7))
 (segment (start 139.7 134.62) (end 142.24 134.62) (width 0.8) (layer F.Cu) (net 7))
 (segment (start 148.59 134.62) (end 149.86 135.89) (width 0.8) (layer F.Cu) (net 7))
 (segment (start 144.78 134.62) (end 148.59 134.62) (width 0.8) (layer F.Cu) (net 7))
 (segment (start 140.97 121.92) (end 142.24 123.19) (width 0.8) (layer F.Cu) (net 7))
 (segment (start 140.97 93.98) (end 140.97 121.92) (width 0.8) (layer F.Cu) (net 7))
 (segment (start 106.68 147.32) (end 102.87 143.51) (width 1.6) (layer F.Cu) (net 8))
 (segment (start 133.35 147.32) (end 106.68 147.32) (width 1.6) (layer F.Cu) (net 8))
 (segment (start 142.4 147.32) (end 144.78 144.94) (width 1.6) (layer F.Cu) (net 8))
 (segment (start 144.78 144.94) (end 144.78 142.24) (width 1.6) (layer F.Cu) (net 8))
 (segment (start 133.35 147.32) (end 142.4 147.32) (width 1.6) (layer F.Cu) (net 8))
 (segment (start 120.65 144.78) (end 128.27 144.78) (width 1.6) (layer F.Cu) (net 9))
 (segment (start 102.87 137.16) (end 113.03 137.16) (width 1.6) (layer F.Cu) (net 9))
 (segment (start 113.03 137.16) (end 120.65 144.78) (width 1.6) (layer F.Cu) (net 9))
 (segment (start 130.87 144.78) (end 133.41 142.24) (width 1.6) (layer F.Cu) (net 9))
 (segment (start 128.27 144.78) (end 130.87 144.78) (width 1.6) (layer F.Cu) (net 9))
 (segment (start 133.41 142.24) (end 139.7 142.24) (width 1.6) (layer F.Cu) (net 9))
 (segment (start 105.41 125.73) (end 114.3 125.73) (width 0.8) (layer F.Cu) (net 10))
 (segment (start 120.65 125.73) (end 121.92 127) (width 0.8) (layer F.Cu) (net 10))
 (segment (start 120.65 125.73) (end 114.3 125.73) (width 0.8) (layer F.Cu) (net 10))
 (segment (start 125.73 116.3) (end 125.19 116.84) (width 0.8) (layer F.Cu) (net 11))
 (segment (start 125.73 114.3) (end 125.73 116.3) (width 0.8) (layer F.Cu) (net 11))
 (segment (start 109.22 116.84) (end 105.41 120.65) (width 0.8) (layer F.Cu) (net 11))
 (segment (start 125.19 116.84) (end 109.22 116.84) (width 0.8) (layer F.Cu) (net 11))
 (segment (start 121.92 137.69) (end 121.92 134.48137) (width 0.8) (layer F.Cu) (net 12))
 (segment (start 121.92 134.48137) (end 121.92 133.35) (width 0.8) (layer F.Cu) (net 12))
 (segment (start 126.47 142.24) (end 121.92 137.69) (width 0.8) (layer F.Cu) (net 12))
 (segment (start 128.27 142.24) (end 126.47 142.24) (width 0.8) (layer F.Cu) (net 12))
 (segment (start 129.54 142.24) (end 133.35 138.43) (width 1.6) (layer F.Cu) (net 12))
 (segment (start 128.27 142.24) (end 129.54 142.24) (width 1.6) (layer F.Cu) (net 12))
 (segment (start 128.27 139.7) (end 128.27 137.16) (width 0.8) (layer F.Cu) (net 13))
 (segment (start 128.27 137.16) (end 125.73 134.62) (width 0.8) (layer F.Cu) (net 13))
 (segment (start 125.73 134.62) (end 125.73 127) (width 0.8) (layer F.Cu) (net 13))
 (segment (start 123.19 124.46) (end 123.19 121.92) (width 0.8) (layer F.Cu) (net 13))
 (segment (start 125.73 127) (end 123.19 124.46) (width 0.8) (layer F.Cu) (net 13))
 (segment (start 115.57 130.81) (end 118.11 133.35) (width 0.8) (layer F.Cu) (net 14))
 (segment (start 102.87 130.81) (end 115.57 130.81) (width 0.8) (layer F.Cu) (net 14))
 (segment (start 138.43 116.84) (end 135.89 119.38) (width 0.8) (layer F.Cu) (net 27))
 (segment (start 135.89 119.38) (end 121.92 119.38) (width 0.8) (layer F.Cu) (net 27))
 (segment (start 121.92 119.38) (end 120.65 120.65) (width 0.8) (layer F.Cu) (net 27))
 (segment (start 120.65 120.65) (end 120.65 121.92) (width 0.8) (layer F.Cu) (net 27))
 (segment (start 119.38 123.19) (end 110.49 123.19) (width 0.8) (layer F.Cu) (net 27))
 (segment (start 120.65 121.92) (end 119.38 123.19) (width 0.8) (layer F.Cu) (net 27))
 (segment (start 119.38 88.9) (end 121.92 91.44) (width 0.8) (layer F.Cu) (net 3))
 (segment (start 121.92 91.44) (end 128.27 91.44) (width 0.8) (layer F.Cu) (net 3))
 (segment (start 128.27 91.44) (end 138.43 91.44) (width 0.8) (layer F.Cu) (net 3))
 (segment (start 128.27 88.9) (end 138.43 88.9) (width 0.8) (layer F.Cu) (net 1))
 (segment (start 124.46 85.09) (end 128.27 88.9) (width 0.8) (layer F.Cu) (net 1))
 (segment (start 138.43 86.36) (end 133.35 86.36) (width 0.8) (layer F.Cu) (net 4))
 (segment (start 128.27 82.55) (end 128.27 78.74) (width 0.8) (layer F.Cu) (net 4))
 (segment (start 132.08 86.36) (end 128.27 82.55) (width 0.8) (layer F.Cu) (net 4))
 (segment (start 132.08 86.36) (end 133.35 86.36) (width 0.8) (layer F.Cu) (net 4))
 (segment (start 108.11 111.72) (end 112.99 111.72) (width 0.8) (layer F.Cu) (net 15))
 (segment (start 115.49 109.22) (end 118.11 109.22) (width 0.8) (layer F.Cu) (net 15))
 (segment (start 112.99 111.72) (end 115.49 109.22) (width 0.8) (layer F.Cu) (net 15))
 (segment (start 118.11 105.41) (end 119.38 104.14) (width 0.8) (layer F.Cu) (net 15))
 (segment (start 118.11 109.22) (end 118.11 105.41) (width 0.8) (layer F.Cu) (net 15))
 (segment (start 106.52 103.98) (end 106.68 104.14) (width 0.8) (layer F.Cu) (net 16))
 (segment (start 102.87 103.98) (end 106.52 103.98) (width 0.8) (layer F.Cu) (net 16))
 (segment (start 133.35 99.06) (end 138.43 99.06) (width 0.8) (layer F.Cu) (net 17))
 (segment (start 133.35 99.06) (end 133.35 101.6) (width 0.8) (layer F.Cu) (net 17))
 (segment (start 125.73 96.52) (end 128.27 96.52) (width 0.8) (layer F.Cu) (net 18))
 (segment (start 123.19 99.06) (end 125.73 96.52) (width 0.8) (layer F.Cu) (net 18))
 (segment (start 123.19 99.06) (end 119.38 99.06) (width 0.8) (layer F.Cu) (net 18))
 (segment (start 128.27 96.52) (end 138.43 96.52) (width 0.8) (layer F.Cu) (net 18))
 (segment (start 102.95 99.06) (end 102.87 98.98) (width 0.8) (layer F.Cu) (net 19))
 (segment (start 106.68 99.06) (end 102.95 99.06) (width 0.8) (layer F.Cu) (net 19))
 (segment (start 146.05 86.36) (end 149.86 82.55) (width 0.8) (layer F.Cu) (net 20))
 (segment (start 152.4 82.55) (end 156.21 78.74) (width 0.8) (layer F.Cu) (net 20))
 (segment (start 149.86 82.55) (end 152.4 82.55) (width 0.8) (layer F.Cu) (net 20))
 (segment (start 156.21 78.74) (end 161.29 78.74) (width 0.8) (layer F.Cu) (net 20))
 (segment (start 156.21 91.44) (end 146.05 91.44) (width 0.8) (layer F.Cu) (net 21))
 (segment (start 142.16 78.78) (end 142.16 82.47) (width 0.8) (layer F.Cu) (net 21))
 (segment (start 142.16 82.47) (end 143.51 83.82) (width 0.8) (layer F.Cu) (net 21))
 (segment (start 145.65 91.44) (end 146.05 91.44) (width 0.8) (layer F.Cu) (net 21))
 (segment (start 143.51 89.3) (end 145.65 91.44) (width 0.8) (layer F.Cu) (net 21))
 (segment (start 143.51 83.82) (end 143.51 89.3) (width 0.8) (layer F.Cu) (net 21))
 (segment (start 102.87 93.98) (end 106.68 93.98) (width 0.8) (layer F.Cu) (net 22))
 (segment (start 138.43 101.6) (end 138.43 106.68) (width 0.8) (layer F.Cu) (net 23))
 (segment (start 137.16 106.68) (end 133.35 110.49) (width 0.8) (layer F.Cu) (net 23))
 (segment (start 138.43 106.68) (end 137.16 106.68) (width 0.8) (layer F.Cu) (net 23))
 (segment (start 133.35 114.3) (end 133.35 110.49) (width 0.8) (layer F.Cu) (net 23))
 (segment (start 153.67 97.79) (end 153.67 101.6) (width 0.8) (layer F.Cu) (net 24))
 (segment (start 152.4 96.52) (end 153.67 97.79) (width 0.8) (layer F.Cu) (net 24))
 (segment (start 153.67 101.6) (end 151.13 104.14) (width 0.8) (layer F.Cu) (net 24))
 (segment (start 151.13 104.14) (end 151.13 106.68) (width 0.8) (layer F.Cu) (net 24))
 (segment (start 152.4 96.52) (end 146.05 96.52) (width 0.8) (layer F.Cu) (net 24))
 (segment (start 151.13 99.06) (end 146.05 99.06) (width 0.8) (layer F.Cu) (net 25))
 (segment (start 146.05 106.68) (end 151.13 111.76) (width 0.8) (layer F.Cu) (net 26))
 (segment (start 146.05 101.6) (end 146.05 106.68) (width 0.8) (layer F.Cu) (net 26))
 (segment (start 151.13 111.76) (end 151.13 116.84) (width 0.8) (layer F.Cu) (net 26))
 (segment (start 128.27 114.7) (end 130.41 116.84) (width 0.8) (layer F.Cu) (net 28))
 (segment (start 128.27 114.3) (end 128.27 114.7) (width 0.8) (layer F.Cu) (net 28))
 (segment (start 134.62 116.84) (end 130.41 116.84) (width 0.8) (layer F.Cu) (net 28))
 (segment (start 138.43 113.03) (end 138.43 111.76) (width 0.8) (layer F.Cu) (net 28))
 (segment (start 138.43 113.03) (end 134.62 116.84) (width 0.8) (layer F.Cu) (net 28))
 (segment (start 128.27 129.54) (end 128.27 121.92) (width 0.8) (layer F.Cu) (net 29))
 (segment (start 132.08 133.35) (end 128.27 129.54) (width 0.8) (layer F.Cu) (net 29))
 (segment (start 132.08 133.35) (end 134.62 133.35) (width 0.8) (layer F.Cu) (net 29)))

